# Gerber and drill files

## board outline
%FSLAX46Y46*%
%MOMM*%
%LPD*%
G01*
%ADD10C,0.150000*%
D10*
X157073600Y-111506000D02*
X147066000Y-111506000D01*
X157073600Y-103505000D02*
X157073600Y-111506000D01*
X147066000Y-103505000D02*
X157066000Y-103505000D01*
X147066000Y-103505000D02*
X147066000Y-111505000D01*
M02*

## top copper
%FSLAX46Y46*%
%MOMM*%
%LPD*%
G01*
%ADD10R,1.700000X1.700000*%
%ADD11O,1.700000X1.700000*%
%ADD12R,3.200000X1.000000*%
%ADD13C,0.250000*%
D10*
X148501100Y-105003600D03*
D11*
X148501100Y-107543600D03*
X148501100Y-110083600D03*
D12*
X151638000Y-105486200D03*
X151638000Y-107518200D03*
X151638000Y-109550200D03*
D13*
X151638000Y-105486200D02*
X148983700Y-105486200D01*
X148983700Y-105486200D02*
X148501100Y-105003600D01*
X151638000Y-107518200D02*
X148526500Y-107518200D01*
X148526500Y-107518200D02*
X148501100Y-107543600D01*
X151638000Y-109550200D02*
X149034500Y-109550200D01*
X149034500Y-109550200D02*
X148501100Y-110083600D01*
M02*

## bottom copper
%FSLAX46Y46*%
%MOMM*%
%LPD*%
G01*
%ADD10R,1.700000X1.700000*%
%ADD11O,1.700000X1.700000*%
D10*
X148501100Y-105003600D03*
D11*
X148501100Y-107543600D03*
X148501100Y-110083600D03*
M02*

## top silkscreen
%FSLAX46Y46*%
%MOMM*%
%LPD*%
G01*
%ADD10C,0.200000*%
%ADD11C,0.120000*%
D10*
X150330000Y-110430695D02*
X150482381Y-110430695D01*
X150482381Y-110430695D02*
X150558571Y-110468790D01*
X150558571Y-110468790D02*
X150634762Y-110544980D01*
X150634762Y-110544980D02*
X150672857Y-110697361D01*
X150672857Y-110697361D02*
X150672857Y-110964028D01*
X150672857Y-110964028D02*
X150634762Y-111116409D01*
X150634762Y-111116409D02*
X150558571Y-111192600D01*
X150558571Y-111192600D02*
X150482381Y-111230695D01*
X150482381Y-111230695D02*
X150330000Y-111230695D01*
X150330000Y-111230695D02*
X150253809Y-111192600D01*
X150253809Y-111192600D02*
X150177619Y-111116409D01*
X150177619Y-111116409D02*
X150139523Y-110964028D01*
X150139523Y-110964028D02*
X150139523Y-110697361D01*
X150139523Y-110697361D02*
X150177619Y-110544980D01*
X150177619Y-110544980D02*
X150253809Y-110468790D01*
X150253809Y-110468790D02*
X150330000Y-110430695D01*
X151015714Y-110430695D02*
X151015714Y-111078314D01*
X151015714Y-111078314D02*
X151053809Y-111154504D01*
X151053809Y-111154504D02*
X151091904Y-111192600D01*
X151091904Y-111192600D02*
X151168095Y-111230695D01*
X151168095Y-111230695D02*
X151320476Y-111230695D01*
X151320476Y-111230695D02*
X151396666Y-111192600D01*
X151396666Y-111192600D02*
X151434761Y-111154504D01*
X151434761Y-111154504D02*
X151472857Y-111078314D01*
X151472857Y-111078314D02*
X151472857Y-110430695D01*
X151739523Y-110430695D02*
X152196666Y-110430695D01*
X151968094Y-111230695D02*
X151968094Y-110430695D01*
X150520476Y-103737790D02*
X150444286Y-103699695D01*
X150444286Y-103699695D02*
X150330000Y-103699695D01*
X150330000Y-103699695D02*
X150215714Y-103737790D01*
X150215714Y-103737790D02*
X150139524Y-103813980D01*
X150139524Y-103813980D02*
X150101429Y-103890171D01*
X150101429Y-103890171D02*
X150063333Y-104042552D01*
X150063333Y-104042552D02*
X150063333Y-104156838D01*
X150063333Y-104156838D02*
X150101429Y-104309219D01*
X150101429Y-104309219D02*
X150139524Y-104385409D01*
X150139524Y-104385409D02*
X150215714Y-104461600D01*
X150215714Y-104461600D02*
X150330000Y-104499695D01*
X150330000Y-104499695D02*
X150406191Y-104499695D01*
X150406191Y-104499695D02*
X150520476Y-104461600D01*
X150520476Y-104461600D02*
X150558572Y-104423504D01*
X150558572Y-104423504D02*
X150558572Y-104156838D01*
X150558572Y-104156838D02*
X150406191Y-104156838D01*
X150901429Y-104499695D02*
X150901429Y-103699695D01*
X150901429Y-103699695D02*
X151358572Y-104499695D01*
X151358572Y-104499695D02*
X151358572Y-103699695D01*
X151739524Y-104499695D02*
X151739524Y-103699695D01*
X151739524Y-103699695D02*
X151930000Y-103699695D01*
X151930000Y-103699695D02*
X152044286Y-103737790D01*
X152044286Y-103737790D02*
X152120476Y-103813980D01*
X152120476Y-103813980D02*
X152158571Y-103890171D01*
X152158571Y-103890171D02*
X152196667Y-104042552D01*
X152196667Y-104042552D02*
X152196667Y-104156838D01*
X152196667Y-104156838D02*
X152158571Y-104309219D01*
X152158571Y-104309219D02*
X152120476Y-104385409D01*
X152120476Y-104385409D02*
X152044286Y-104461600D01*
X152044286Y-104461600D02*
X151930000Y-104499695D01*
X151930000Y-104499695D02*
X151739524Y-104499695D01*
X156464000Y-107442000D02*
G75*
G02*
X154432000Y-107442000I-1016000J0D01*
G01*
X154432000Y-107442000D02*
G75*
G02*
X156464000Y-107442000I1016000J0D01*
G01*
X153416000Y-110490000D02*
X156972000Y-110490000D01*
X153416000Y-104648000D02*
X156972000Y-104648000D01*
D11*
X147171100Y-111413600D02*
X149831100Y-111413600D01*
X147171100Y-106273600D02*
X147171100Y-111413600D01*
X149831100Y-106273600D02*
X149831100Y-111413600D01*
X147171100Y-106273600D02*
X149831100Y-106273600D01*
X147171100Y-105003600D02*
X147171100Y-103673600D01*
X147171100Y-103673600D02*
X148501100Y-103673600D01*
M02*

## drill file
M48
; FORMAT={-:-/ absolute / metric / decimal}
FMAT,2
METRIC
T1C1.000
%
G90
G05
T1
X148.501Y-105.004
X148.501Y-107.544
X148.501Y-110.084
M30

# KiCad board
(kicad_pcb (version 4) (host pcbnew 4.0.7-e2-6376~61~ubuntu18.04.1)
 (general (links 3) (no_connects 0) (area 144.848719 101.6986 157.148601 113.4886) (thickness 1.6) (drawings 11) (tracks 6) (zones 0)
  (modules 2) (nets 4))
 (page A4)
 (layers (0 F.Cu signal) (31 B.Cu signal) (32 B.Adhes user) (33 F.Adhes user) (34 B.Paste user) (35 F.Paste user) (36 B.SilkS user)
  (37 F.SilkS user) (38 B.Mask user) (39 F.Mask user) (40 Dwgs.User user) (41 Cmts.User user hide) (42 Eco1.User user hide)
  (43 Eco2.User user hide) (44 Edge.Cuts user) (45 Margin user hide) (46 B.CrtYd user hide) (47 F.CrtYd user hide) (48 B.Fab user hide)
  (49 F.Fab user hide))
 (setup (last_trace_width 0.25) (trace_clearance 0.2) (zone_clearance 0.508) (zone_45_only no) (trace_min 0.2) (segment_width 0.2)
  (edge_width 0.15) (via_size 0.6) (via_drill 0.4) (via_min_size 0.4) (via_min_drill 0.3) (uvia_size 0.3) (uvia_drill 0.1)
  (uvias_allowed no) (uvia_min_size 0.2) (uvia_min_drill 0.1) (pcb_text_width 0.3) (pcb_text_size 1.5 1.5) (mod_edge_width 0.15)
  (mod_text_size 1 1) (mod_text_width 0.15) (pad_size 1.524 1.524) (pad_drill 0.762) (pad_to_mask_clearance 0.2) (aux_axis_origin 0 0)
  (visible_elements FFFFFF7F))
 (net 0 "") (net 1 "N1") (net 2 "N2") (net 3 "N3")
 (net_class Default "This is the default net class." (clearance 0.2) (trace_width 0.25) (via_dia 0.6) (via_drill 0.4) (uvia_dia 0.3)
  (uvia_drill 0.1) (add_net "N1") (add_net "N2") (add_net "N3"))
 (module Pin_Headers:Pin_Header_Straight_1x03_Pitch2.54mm (layer F.Cu) (at 148.5011 105.0036)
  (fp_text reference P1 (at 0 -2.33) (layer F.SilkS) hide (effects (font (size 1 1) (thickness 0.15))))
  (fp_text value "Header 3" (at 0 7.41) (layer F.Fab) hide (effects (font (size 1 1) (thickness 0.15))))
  (fp_line (start -1.33 6.41) (end 1.33 6.41) (layer F.SilkS) (width 0.12))
  (fp_line (start -1.33 1.27) (end -1.33 6.41) (layer F.SilkS) (width 0.12))
  (fp_line (start 1.33 1.27) (end 1.33 6.41) (layer F.SilkS) (width 0.12))
  (fp_line (start -1.33 1.27) (end 1.33 1.27) (layer F.SilkS) (width 0.12))
  (fp_line (start -1.33 0) (end -1.33 -1.33) (layer F.SilkS) (width 0.12))
  (fp_line (start -1.33 -1.33) (end 0 -1.33) (layer F.SilkS) (width 0.12))
  (pad 1 thru_hole rect (at 0 0) (size 1.7 1.7) (drill 1) (layers *.Cu *.Mask) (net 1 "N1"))
  (pad 2 thru_hole oval (at 0 2.54) (size 1.7 1.7) (drill 1) (layers *.Cu *.Mask) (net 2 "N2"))
  (pad 3 thru_hole oval (at 0 5.08) (size 1.7 1.7) (drill 1) (layers *.Cu *.Mask) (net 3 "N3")))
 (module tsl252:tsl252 (layer F.Cu) (at 153.162 109.0422 90)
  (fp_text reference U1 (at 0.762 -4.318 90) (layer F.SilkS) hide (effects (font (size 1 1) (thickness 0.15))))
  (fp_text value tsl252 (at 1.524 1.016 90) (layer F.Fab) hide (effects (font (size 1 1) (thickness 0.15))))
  (pad 3 smd rect (at 3.556 -1.524 90) (size 1 3.2) (layers F.Cu F.Paste F.Mask) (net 1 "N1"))
  (pad 2 smd rect (at 1.524 -1.524 90) (size 1 3.2) (layers F.Cu F.Paste F.Mask) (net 2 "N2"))
  (pad 1 smd rect (at -0.508 -1.524 90) (size 1 3.2) (layers F.Cu F.Paste F.Mask) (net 3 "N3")))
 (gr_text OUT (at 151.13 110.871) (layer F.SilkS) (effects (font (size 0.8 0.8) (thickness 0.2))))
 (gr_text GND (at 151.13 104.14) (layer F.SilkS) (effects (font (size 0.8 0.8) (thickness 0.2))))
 (gr_circle (center 155.448 107.442) (end 155.448 108.458) (layer F.SilkS) (width 0.2))
 (gr_line (start 153.416 110.49) (end 156.972 110.49) (angle 90) (layer F.SilkS) (width 0.2))
 (gr_line (start 153.416 104.648) (end 156.972 104.648) (angle 90) (layer F.SilkS) (width 0.2))
 (gr_line (start 157.0736 111.506) (end 147.066 111.506) (angle 90) (layer Edge.Cuts) (width 0.15))
 (gr_line (start 157.0736 103.505) (end 157.0736 111.506) (angle 90) (layer Edge.Cuts) (width 0.15))
 (gr_line (start 147.066 103.505) (end 157.066 103.505) (angle 90) (layer Edge.Cuts) (width 0.15))
 (gr_line (start 147.066 103.505) (end 147.066 111.505) (angle 90) (layer Edge.Cuts) (width 0.15))
 (segment (start 151.638 105.4862) (end 148.9837 105.4862) (width 0.25) (layer F.Cu) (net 1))
 (segment (start 148.9837 105.4862) (end 148.5011 105.0036) (width 0.25) (layer F.Cu) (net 1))
 (segment (start 151.638 107.5182) (end 148.5265 107.5182) (width 0.25) (layer F.Cu) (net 2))
 (segment (start 148.5265 107.5182) (end 148.5011 107.5436) (width 0.25) (layer F.Cu) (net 2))
 (segment (start 151.638 109.5502) (end 149.0345 109.5502) (width 0.25) (layer F.Cu) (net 3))
 (segment (start 149.0345 109.5502) (end 148.5011 110.0836) (width 0.25) (layer F.Cu) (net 3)))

